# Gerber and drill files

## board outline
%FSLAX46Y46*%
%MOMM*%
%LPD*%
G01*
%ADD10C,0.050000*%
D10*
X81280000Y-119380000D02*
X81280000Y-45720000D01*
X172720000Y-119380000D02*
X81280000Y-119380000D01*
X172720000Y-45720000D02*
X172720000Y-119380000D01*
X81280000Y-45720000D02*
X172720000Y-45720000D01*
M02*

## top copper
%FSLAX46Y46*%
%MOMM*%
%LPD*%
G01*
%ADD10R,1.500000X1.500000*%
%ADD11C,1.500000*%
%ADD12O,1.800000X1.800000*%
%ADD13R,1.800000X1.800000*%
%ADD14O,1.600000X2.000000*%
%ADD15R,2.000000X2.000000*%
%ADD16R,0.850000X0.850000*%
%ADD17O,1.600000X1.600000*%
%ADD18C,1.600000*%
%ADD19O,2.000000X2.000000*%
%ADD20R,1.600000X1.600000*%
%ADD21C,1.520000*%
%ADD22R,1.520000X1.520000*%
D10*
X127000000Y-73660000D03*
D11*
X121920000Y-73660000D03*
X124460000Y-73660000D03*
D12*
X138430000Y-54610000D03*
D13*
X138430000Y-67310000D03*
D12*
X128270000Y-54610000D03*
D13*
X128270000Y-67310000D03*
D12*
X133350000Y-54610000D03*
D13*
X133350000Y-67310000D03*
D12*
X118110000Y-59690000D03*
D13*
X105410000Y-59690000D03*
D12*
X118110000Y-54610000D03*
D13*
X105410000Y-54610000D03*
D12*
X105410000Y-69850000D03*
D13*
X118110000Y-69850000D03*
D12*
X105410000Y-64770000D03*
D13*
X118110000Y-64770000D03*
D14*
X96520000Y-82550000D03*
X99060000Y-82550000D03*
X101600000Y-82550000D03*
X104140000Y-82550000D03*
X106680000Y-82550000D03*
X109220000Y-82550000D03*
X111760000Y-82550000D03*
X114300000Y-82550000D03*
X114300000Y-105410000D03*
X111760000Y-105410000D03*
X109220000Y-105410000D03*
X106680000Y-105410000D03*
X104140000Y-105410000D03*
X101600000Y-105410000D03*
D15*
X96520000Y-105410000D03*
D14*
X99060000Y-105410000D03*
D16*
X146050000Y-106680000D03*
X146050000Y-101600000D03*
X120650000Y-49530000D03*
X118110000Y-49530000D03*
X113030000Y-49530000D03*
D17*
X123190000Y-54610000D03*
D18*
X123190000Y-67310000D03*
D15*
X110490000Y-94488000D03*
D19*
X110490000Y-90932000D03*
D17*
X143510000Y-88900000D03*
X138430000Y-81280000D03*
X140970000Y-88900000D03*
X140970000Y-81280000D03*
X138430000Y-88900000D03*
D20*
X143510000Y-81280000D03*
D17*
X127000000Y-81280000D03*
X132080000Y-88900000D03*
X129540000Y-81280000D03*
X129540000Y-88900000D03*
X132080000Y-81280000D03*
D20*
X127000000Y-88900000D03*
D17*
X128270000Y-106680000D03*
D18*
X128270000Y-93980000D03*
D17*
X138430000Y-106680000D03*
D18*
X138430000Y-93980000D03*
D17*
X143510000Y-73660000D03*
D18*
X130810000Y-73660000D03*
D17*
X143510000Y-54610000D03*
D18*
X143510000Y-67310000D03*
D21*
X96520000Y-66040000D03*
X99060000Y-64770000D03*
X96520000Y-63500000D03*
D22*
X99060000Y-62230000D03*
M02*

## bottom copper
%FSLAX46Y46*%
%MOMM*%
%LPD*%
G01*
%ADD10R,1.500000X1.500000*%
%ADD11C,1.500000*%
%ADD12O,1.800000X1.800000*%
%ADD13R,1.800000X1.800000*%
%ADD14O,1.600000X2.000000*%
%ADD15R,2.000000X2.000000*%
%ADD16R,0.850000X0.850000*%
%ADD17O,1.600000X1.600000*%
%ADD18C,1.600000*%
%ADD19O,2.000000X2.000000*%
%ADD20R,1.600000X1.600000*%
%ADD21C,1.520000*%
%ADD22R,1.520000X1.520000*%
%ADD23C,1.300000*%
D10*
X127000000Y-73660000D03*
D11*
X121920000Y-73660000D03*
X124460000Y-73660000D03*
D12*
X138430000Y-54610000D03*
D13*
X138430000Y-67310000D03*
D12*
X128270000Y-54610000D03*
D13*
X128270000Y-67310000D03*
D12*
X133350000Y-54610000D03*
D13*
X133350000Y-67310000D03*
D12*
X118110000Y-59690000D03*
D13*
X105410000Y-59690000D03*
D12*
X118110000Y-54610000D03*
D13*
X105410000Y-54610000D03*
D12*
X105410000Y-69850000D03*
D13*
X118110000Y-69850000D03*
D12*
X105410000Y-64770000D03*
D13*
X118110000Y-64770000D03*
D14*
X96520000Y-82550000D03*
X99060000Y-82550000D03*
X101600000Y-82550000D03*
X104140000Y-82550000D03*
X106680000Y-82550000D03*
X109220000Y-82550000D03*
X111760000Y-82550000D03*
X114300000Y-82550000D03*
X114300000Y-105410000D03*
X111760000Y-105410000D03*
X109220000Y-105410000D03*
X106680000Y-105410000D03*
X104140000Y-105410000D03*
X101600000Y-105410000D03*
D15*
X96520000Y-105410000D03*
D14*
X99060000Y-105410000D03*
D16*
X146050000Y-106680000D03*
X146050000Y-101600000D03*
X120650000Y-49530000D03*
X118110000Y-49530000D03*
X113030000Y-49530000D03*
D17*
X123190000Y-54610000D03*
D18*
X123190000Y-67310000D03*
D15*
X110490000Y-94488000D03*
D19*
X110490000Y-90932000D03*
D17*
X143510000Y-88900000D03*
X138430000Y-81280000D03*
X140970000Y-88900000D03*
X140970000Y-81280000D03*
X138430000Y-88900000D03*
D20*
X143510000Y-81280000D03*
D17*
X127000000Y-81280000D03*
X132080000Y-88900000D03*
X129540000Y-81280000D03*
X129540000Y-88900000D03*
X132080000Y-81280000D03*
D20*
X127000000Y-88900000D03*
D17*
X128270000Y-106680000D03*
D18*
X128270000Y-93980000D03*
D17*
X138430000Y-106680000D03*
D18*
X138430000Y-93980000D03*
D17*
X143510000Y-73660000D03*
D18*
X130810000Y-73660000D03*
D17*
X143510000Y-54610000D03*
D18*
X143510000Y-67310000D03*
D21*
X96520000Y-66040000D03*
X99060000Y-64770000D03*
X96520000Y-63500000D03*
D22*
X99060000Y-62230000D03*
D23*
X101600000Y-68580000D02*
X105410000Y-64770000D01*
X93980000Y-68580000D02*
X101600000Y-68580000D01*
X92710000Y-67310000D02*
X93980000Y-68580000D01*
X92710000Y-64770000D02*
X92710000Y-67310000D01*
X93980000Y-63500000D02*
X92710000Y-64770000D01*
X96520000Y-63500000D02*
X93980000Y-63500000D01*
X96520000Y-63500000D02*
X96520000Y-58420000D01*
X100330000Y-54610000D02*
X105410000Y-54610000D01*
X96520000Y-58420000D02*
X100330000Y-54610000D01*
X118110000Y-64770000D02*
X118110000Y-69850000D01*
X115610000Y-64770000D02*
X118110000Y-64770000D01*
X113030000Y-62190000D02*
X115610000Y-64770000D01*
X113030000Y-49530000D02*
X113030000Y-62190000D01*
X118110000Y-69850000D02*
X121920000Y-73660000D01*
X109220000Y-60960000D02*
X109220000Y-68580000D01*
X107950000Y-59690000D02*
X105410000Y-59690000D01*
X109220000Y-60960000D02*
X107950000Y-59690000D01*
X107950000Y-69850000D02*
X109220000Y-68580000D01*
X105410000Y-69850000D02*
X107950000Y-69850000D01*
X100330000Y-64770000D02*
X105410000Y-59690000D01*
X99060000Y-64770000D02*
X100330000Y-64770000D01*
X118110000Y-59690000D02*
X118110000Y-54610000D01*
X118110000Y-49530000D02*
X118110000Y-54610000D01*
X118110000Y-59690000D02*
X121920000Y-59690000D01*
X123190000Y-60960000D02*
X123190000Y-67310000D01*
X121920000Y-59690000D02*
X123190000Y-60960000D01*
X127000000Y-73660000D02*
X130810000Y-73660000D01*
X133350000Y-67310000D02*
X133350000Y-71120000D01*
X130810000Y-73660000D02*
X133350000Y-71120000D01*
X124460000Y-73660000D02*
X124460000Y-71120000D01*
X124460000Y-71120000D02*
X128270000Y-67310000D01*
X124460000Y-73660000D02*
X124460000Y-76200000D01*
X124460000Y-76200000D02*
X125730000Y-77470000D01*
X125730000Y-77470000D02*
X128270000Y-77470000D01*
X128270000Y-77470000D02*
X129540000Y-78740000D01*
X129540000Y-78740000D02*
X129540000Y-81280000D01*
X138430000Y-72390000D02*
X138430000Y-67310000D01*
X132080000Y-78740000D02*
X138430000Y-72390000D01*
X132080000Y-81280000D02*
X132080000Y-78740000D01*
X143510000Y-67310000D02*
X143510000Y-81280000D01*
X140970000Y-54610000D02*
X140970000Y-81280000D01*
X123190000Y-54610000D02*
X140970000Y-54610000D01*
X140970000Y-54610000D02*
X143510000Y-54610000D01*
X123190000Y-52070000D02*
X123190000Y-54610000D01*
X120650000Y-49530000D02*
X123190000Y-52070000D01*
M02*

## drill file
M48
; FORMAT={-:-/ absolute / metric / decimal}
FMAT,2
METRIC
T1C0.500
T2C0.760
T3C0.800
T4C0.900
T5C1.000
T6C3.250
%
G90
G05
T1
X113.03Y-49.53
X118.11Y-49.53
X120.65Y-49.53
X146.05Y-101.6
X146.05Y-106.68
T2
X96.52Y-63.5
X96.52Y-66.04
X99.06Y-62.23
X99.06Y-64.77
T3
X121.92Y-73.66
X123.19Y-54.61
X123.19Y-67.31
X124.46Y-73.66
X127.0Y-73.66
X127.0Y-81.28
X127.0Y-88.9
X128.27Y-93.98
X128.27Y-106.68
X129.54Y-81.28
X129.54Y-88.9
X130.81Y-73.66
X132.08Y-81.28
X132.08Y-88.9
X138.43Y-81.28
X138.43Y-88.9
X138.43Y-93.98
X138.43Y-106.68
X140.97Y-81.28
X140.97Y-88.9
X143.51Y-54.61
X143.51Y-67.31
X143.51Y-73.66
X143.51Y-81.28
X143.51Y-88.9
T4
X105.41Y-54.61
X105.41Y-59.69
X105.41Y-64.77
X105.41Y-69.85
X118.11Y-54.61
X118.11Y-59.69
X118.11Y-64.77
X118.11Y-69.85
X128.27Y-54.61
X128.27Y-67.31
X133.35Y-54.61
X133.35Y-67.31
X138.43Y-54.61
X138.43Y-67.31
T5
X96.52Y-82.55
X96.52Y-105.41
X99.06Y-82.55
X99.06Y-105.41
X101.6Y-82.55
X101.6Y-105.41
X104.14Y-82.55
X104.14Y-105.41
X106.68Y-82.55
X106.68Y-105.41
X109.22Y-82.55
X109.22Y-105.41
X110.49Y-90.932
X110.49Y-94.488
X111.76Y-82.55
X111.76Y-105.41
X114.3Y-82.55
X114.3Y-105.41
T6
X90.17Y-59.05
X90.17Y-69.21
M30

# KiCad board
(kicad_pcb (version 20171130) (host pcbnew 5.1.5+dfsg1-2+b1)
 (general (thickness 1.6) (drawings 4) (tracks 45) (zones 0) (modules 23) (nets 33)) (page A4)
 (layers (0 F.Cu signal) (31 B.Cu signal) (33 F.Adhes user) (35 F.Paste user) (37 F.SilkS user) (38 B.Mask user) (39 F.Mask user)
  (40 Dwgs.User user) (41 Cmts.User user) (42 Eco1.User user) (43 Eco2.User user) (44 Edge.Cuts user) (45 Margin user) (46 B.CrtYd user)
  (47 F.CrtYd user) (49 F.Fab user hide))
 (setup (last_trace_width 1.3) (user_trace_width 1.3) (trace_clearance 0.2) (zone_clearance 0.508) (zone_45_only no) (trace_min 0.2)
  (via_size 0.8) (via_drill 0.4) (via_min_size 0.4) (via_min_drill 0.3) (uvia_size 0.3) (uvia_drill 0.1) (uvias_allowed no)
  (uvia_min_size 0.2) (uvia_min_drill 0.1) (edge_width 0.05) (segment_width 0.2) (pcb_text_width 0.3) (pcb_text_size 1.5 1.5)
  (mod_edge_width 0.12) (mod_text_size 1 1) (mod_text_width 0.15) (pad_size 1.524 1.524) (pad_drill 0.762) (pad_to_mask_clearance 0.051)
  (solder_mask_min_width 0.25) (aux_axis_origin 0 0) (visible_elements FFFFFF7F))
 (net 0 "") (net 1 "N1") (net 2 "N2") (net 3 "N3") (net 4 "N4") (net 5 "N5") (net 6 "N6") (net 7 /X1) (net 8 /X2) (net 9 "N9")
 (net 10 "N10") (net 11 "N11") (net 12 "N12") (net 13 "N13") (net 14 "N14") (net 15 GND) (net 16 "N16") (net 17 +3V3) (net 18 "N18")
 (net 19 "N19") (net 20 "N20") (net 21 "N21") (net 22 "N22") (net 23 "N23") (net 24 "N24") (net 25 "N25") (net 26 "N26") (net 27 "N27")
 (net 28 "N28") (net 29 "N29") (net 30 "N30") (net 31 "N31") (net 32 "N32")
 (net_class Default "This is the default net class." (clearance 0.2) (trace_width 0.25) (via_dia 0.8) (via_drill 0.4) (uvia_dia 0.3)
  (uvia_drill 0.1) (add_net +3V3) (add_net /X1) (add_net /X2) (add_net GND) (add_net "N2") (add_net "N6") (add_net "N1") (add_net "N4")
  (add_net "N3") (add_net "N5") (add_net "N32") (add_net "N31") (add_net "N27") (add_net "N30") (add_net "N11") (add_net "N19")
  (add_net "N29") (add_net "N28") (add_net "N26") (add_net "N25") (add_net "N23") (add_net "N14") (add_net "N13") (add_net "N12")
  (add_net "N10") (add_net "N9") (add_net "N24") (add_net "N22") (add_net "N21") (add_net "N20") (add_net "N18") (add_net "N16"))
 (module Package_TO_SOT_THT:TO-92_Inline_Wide (layer F.Cu) (at 127 73.66 180)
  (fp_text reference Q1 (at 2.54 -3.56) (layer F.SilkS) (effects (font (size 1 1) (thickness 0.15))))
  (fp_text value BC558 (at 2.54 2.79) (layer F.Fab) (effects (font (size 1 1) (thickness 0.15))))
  (pad 1 thru_hole rect (at 0 0 270) (size 1.5 1.5) (drill 0.8) (layers *.Cu *.Mask) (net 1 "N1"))
  (pad 3 thru_hole circle (at 5.08 0 270) (size 1.5 1.5) (drill 0.8) (layers *.Cu *.Mask) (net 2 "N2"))
  (pad 2 thru_hole circle (at 2.54 0 270) (size 1.5 1.5) (drill 0.8) (layers *.Cu *.Mask) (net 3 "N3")))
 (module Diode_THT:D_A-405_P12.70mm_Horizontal (layer F.Cu) (at 138.43 67.31 90)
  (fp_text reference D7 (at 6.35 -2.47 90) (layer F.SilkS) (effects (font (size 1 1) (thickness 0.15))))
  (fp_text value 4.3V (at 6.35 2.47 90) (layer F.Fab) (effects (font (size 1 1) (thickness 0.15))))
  (pad 2 thru_hole oval (at 12.7 0 90) (size 1.8 1.8) (drill 0.9) (layers *.Cu *.Mask) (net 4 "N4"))
  (pad 1 thru_hole rect (at 0 0 90) (size 1.8 1.8) (drill 0.9) (layers *.Cu *.Mask) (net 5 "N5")))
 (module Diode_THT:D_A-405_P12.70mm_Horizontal (layer F.Cu) (at 128.27 67.31 90)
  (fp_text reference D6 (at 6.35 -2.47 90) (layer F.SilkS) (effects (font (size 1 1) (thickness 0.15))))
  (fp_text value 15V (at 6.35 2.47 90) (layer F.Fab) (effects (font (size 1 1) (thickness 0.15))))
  (pad 2 thru_hole oval (at 12.7 0 90) (size 1.8 1.8) (drill 0.9) (layers *.Cu *.Mask) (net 4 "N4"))
  (pad 1 thru_hole rect (at 0 0 90) (size 1.8 1.8) (drill 0.9) (layers *.Cu *.Mask) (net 3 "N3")))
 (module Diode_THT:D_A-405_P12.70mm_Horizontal (layer F.Cu) (at 133.35 67.31 90)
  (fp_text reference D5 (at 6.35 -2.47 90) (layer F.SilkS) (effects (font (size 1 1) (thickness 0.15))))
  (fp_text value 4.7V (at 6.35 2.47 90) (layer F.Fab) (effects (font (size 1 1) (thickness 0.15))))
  (pad 2 thru_hole oval (at 12.7 0 90) (size 1.8 1.8) (drill 0.9) (layers *.Cu *.Mask) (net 4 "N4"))
  (pad 1 thru_hole rect (at 0 0 90) (size 1.8 1.8) (drill 0.9) (layers *.Cu *.Mask) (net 1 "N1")))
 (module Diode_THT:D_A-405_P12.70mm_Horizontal (layer F.Cu) (at 105.41 59.69)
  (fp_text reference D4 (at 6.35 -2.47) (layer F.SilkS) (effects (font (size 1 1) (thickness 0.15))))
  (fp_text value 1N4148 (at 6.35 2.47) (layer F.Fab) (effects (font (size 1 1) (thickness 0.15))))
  (pad 2 thru_hole oval (at 12.7 0) (size 1.8 1.8) (drill 0.9) (layers *.Cu *.Mask) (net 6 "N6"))
  (pad 1 thru_hole rect (at 0 0) (size 1.8 1.8) (drill 0.9) (layers *.Cu *.Mask) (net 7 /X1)))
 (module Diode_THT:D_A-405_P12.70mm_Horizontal (layer F.Cu) (at 105.41 54.61)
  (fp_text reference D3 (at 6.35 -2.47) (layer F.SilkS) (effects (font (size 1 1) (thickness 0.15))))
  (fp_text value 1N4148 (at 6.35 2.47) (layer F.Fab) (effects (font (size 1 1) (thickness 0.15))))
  (pad 2 thru_hole oval (at 12.7 0) (size 1.8 1.8) (drill 0.9) (layers *.Cu *.Mask) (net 6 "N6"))
  (pad 1 thru_hole rect (at 0 0) (size 1.8 1.8) (drill 0.9) (layers *.Cu *.Mask) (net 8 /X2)))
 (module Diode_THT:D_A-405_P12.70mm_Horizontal (layer F.Cu) (at 118.11 69.85 180)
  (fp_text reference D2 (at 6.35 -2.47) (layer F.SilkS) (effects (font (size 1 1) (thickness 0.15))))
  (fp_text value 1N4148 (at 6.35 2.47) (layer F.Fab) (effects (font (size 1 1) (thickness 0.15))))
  (pad 2 thru_hole oval (at 12.7 0 180) (size 1.8 1.8) (drill 0.9) (layers *.Cu *.Mask) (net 7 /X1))
  (pad 1 thru_hole rect (at 0 0 180) (size 1.8 1.8) (drill 0.9) (layers *.Cu *.Mask) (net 2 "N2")))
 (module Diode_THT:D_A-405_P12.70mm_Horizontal (layer F.Cu) (at 118.11 64.77 180)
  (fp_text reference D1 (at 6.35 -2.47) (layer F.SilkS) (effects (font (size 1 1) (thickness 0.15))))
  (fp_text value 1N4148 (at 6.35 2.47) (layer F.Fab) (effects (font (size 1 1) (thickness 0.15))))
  (pad 2 thru_hole oval (at 12.7 0 180) (size 1.8 1.8) (drill 0.9) (layers *.Cu *.Mask) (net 8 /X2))
  (pad 1 thru_hole rect (at 0 0 180) (size 1.8 1.8) (drill 0.9) (layers *.Cu *.Mask) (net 2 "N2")))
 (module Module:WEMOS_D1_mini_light (layer F.Cu) (at 96.52 105.41 90)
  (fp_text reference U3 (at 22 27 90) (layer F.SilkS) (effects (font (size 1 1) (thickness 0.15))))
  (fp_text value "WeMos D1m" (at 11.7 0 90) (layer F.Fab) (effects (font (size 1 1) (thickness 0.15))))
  (pad 16 thru_hole oval (at 22.86 0 90) (size 2 1.6) (drill 1) (layers *.Cu *.Mask) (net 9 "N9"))
  (pad 15 thru_hole oval (at 22.86 2.54 90) (size 2 1.6) (drill 1) (layers *.Cu *.Mask) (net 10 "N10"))
  (pad 14 thru_hole oval (at 22.86 5.08 90) (size 2 1.6) (drill 1) (layers *.Cu *.Mask) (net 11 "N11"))
  (pad 13 thru_hole oval (at 22.86 7.62 90) (size 2 1.6) (drill 1) (layers *.Cu *.Mask) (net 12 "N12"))
  (pad 12 thru_hole oval (at 22.86 10.16 90) (size 2 1.6) (drill 1) (layers *.Cu *.Mask) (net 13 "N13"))
  (pad 11 thru_hole oval (at 22.86 12.7 90) (size 2 1.6) (drill 1) (layers *.Cu *.Mask) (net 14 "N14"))
  (pad 10 thru_hole oval (at 22.86 15.24 90) (size 2 1.6) (drill 1) (layers *.Cu *.Mask) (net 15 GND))
  (pad 9 thru_hole oval (at 22.86 17.78 90) (size 2 1.6) (drill 1) (layers *.Cu *.Mask) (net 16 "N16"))
  (pad 8 thru_hole oval (at 0 17.78 90) (size 2 1.6) (drill 1) (layers *.Cu *.Mask) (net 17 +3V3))
  (pad 7 thru_hole oval (at 0 15.24 90) (size 2 1.6) (drill 1) (layers *.Cu *.Mask) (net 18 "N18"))
  (pad 6 thru_hole oval (at 0 12.7 90) (size 2 1.6) (drill 1) (layers *.Cu *.Mask) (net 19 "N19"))
  (pad 5 thru_hole oval (at 0 10.16 90) (size 2 1.6) (drill 1) (layers *.Cu *.Mask) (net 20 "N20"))
  (pad 4 thru_hole oval (at 0 7.62 90) (size 2 1.6) (drill 1) (layers *.Cu *.Mask) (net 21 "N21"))
  (pad 3 thru_hole oval (at 0 5.08 90) (size 2 1.6) (drill 1) (layers *.Cu *.Mask) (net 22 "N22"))
  (pad 1 thru_hole rect (at 0 0 90) (size 2 2) (drill 1) (layers *.Cu *.Mask) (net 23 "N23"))
  (pad 2 thru_hole oval (at 0 2.54 90) (size 2 1.6) (drill 1) (layers *.Cu *.Mask) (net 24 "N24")))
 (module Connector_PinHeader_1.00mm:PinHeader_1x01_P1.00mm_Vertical (layer F.Cu) (at 146.05 106.68)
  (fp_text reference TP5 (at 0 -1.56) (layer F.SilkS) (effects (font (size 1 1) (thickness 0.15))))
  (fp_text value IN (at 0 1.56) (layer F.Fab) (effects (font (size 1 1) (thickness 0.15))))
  (pad 1 thru_hole rect (at 0 0) (size 0.85 0.85) (drill 0.5) (layers *.Cu *.Mask) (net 19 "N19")))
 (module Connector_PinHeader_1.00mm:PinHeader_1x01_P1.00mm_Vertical (layer F.Cu) (at 146.05 101.6)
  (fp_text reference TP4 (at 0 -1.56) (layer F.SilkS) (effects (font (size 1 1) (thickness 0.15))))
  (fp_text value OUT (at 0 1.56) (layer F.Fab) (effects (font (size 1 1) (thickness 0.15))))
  (pad 1 thru_hole rect (at 0 0) (size 0.85 0.85) (drill 0.5) (layers *.Cu *.Mask) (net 11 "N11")))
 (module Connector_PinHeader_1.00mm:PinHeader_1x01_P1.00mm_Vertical (layer F.Cu) (at 120.65 49.53)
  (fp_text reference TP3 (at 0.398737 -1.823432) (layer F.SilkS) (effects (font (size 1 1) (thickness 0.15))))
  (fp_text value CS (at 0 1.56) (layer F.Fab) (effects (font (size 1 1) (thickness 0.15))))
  (pad 1 thru_hole rect (at 0 0) (size 0.85 0.85) (drill 0.5) (layers *.Cu *.Mask) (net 4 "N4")))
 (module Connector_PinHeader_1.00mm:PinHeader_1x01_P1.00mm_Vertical (layer F.Cu) (at 118.11 49.53)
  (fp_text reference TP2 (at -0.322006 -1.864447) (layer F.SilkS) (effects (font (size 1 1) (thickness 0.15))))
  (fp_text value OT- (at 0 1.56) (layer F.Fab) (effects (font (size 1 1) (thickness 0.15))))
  (pad 1 thru_hole rect (at 0 0) (size 0.85 0.85) (drill 0.5) (layers *.Cu *.Mask) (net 6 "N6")))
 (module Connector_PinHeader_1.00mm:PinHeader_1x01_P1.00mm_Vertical (layer F.Cu) (at 113.03 49.53)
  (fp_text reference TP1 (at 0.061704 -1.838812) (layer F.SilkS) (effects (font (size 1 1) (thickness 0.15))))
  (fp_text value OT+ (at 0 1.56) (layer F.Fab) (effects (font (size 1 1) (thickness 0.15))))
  (pad 1 thru_hole rect (at 0 0) (size 0.85 0.85) (drill 0.5) (layers *.Cu *.Mask) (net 2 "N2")))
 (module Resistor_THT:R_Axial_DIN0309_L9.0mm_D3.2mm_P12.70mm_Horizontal (layer F.Cu) (at 123.19 67.31 90)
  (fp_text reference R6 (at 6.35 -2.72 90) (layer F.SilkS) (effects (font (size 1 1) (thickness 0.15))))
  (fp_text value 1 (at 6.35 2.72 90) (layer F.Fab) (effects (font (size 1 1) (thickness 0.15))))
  (pad 2 thru_hole oval (at 12.7 0 90) (size 1.6 1.6) (drill 0.8) (layers *.Cu *.Mask) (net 4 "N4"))
  (pad 1 thru_hole circle (at 0 0 90) (size 1.6 1.6) (drill 0.8) (layers *.Cu *.Mask) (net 6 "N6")))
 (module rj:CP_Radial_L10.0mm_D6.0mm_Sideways (layer F.Cu) (at 110.49 92.71 180)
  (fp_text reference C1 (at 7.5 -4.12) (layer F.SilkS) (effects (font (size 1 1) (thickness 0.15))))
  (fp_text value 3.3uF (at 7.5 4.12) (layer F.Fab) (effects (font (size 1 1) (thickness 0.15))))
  (pad 1 thru_hole rect (at 0 -1.778 180) (size 2 2) (drill 1) (layers *.Cu *.Mask) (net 17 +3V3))
  (pad 2 thru_hole oval (at 0 1.778 180) (size 2 2) (drill 1) (layers *.Cu *.Mask) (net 15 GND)))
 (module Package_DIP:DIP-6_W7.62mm (layer F.Cu) (at 143.51 81.28 270)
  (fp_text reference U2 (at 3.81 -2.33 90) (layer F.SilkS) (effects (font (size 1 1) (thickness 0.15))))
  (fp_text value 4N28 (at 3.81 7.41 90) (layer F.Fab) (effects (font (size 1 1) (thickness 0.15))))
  (pad 6 thru_hole oval (at 7.62 0 270) (size 1.6 1.6) (drill 0.8) (layers *.Cu *.Mask) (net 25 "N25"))
  (pad 3 thru_hole oval (at 0 5.08 270) (size 1.6 1.6) (drill 0.8) (layers *.Cu *.Mask) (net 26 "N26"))
  (pad 5 thru_hole oval (at 7.62 2.54 270) (size 1.6 1.6) (drill 0.8) (layers *.Cu *.Mask) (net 17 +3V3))
  (pad 2 thru_hole oval (at 0 2.54 270) (size 1.6 1.6) (drill 0.8) (layers *.Cu *.Mask) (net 4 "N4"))
  (pad 4 thru_hole oval (at 7.62 5.08 270) (size 1.6 1.6) (drill 0.8) (layers *.Cu *.Mask) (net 19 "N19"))
  (pad 1 thru_hole rect (at 0 0 270) (size 1.6 1.6) (drill 0.8) (layers *.Cu *.Mask) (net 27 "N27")))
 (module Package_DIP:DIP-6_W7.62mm (layer F.Cu) (at 127 88.9 90)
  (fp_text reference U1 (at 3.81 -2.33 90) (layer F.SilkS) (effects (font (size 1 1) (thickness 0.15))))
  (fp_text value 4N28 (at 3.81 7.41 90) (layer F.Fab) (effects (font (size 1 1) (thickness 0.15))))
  (pad 6 thru_hole oval (at 7.62 0 90) (size 1.6 1.6) (drill 0.8) (layers *.Cu *.Mask) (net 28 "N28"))
  (pad 3 thru_hole oval (at 0 5.08 90) (size 1.6 1.6) (drill 0.8) (layers *.Cu *.Mask) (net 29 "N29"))
  (pad 5 thru_hole oval (at 7.62 2.54 90) (size 1.6 1.6) (drill 0.8) (layers *.Cu *.Mask) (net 3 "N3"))
  (pad 2 thru_hole oval (at 0 2.54 90) (size 1.6 1.6) (drill 0.8) (layers *.Cu *.Mask) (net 15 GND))
  (pad 4 thru_hole oval (at 7.62 5.08 90) (size 1.6 1.6) (drill 0.8) (layers *.Cu *.Mask) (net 5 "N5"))
  (pad 1 thru_hole rect (at 0 0 90) (size 1.6 1.6) (drill 0.8) (layers *.Cu *.Mask) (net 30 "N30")))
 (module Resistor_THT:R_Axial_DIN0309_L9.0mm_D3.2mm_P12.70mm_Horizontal (layer F.Cu) (at 128.27 93.98 270)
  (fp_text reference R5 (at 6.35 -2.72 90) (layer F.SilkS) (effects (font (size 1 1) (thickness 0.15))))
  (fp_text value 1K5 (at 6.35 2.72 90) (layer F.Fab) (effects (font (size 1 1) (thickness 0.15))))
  (pad 2 thru_hole oval (at 12.7 0 270) (size 1.6 1.6) (drill 0.8) (layers *.Cu *.Mask) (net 19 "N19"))
  (pad 1 thru_hole circle (at 0 0 270) (size 1.6 1.6) (drill 0.8) (layers *.Cu *.Mask) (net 15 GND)))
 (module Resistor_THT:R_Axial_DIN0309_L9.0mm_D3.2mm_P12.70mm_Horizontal (layer F.Cu) (at 138.43 93.98 270)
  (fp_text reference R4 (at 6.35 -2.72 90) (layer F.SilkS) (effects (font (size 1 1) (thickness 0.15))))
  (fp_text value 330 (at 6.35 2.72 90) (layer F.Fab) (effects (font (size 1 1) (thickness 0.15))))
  (pad 2 thru_hole oval (at 12.7 0 270) (size 1.6 1.6) (drill 0.8) (layers *.Cu *.Mask) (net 11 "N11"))
  (pad 1 thru_hole circle (at 0 0 270) (size 1.6 1.6) (drill 0.8) (layers *.Cu *.Mask) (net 30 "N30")))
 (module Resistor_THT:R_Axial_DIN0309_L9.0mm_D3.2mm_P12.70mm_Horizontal (layer F.Cu) (at 130.81 73.66)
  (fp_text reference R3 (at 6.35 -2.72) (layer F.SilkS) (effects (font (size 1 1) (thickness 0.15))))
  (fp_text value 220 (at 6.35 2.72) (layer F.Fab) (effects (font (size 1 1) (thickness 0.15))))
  (pad 2 thru_hole oval (at 12.7 0) (size 1.6 1.6) (drill 0.8) (layers *.Cu *.Mask) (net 27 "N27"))
  (pad 1 thru_hole circle (at 0 0) (size 1.6 1.6) (drill 0.8) (layers *.Cu *.Mask) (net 1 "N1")))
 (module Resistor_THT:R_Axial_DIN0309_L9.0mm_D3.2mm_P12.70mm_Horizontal (layer F.Cu) (at 143.51 67.31 90)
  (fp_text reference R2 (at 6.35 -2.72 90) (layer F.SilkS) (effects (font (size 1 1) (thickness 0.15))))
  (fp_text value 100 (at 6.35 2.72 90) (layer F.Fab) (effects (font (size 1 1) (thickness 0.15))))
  (pad 2 thru_hole oval (at 12.7 0 90) (size 1.6 1.6) (drill 0.8) (layers *.Cu *.Mask) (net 4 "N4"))
  (pad 1 thru_hole circle (at 0 0 90) (size 1.6 1.6) (drill 0.8) (layers *.Cu *.Mask) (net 27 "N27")))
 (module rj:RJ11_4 (layer F.Cu) (at 99.06 60.96 270)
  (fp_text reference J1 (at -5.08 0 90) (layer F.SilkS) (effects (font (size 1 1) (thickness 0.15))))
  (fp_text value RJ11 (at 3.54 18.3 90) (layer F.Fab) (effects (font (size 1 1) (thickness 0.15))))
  (pad "" np_thru_hole circle (at 8.25 8.89 270) (size 3.25 3.25) (drill 3.25) (layers *.Cu *.Mask))
  (pad 4 thru_hole circle (at 5.08 2.54 270) (size 1.52 1.52) (drill 0.76) (layers *.Cu *.Mask) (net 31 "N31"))
  (pad 3 thru_hole circle (at 3.81 0 270) (size 1.52 1.52) (drill 0.76) (layers *.Cu *.Mask) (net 7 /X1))
  (pad 2 thru_hole circle (at 2.54 2.54 270) (size 1.52 1.52) (drill 0.76) (layers *.Cu *.Mask) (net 8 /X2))
  (pad "" np_thru_hole circle (at -1.91 8.89 270) (size 3.25 3.25) (drill 3.25) (layers *.Cu *.Mask))
  (pad 1 thru_hole rect (at 1.27 0 270) (size 1.52 1.52) (drill 0.76) (layers *.Cu *.Mask) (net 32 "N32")))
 (gr_line (start 81.28 119.38) (end 81.28 45.72) (layer Edge.Cuts) (width 0.05))
 (gr_line (start 172.72 119.38) (end 81.28 119.38) (layer Edge.Cuts) (width 0.05))
 (gr_line (start 172.72 45.72) (end 172.72 119.38) (layer Edge.Cuts) (width 0.05))
 (gr_line (start 81.28 45.72) (end 172.72 45.72) (layer Edge.Cuts) (width 0.05))
 (segment (start 101.6 68.58) (end 105.41 64.77) (width 1.3) (layer B.Cu) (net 8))
 (segment (start 93.98 68.58) (end 101.6 68.58) (width 1.3) (layer B.Cu) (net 8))
 (segment (start 92.71 67.31) (end 93.98 68.58) (width 1.3) (layer B.Cu) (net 8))
 (segment (start 92.71 64.77) (end 92.71 67.31) (width 1.3) (layer B.Cu) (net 8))
 (segment (start 93.98 63.5) (end 92.71 64.77) (width 1.3) (layer B.Cu) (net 8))
 (segment (start 96.52 63.5) (end 93.98 63.5) (width 1.3) (layer B.Cu) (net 8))
 (segment (start 96.52 63.5) (end 96.52 58.42) (width 1.3) (layer B.Cu) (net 8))
 (segment (start 100.33 54.61) (end 105.41 54.61) (width 1.3) (layer B.Cu) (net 8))
 (segment (start 96.52 58.42) (end 100.33 54.61) (width 1.3) (layer B.Cu) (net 8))
 (segment (start 118.11 64.77) (end 118.11 69.85) (width 1.3) (layer B.Cu) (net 2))
 (segment (start 115.61 64.77) (end 118.11 64.77) (width 1.3) (layer B.Cu) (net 2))
 (segment (start 113.03 62.19) (end 115.61 64.77) (width 1.3) (layer B.Cu) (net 2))
 (segment (start 113.03 49.53) (end 113.03 62.19) (width 1.3) (layer B.Cu) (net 2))
 (segment (start 118.11 69.85) (end 121.92 73.66) (width 1.3) (layer B.Cu) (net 2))
 (segment (start 109.22 60.96) (end 109.22 68.58) (width 1.3) (layer B.Cu) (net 7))
 (segment (start 107.95 59.69) (end 105.41 59.69) (width 1.3) (layer B.Cu) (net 7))
 (segment (start 109.22 60.96) (end 107.95 59.69) (width 1.3) (layer B.Cu) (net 7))
 (segment (start 107.95 69.85) (end 109.22 68.58) (width 1.3) (layer B.Cu) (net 7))
 (segment (start 105.41 69.85) (end 107.95 69.85) (width 1.3) (layer B.Cu) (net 7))
 (segment (start 100.33 64.77) (end 105.41 59.69) (width 1.3) (layer B.Cu) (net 7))
 (segment (start 99.06 64.77) (end 100.33 64.77) (width 1.3) (layer B.Cu) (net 7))
 (segment (start 118.11 59.69) (end 118.11 54.61) (width 1.3) (layer B.Cu) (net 6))
 (segment (start 118.11 49.53) (end 118.11 54.61) (width 1.3) (layer B.Cu) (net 6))
 (segment (start 118.11 59.69) (end 121.92 59.69) (width 1.3) (layer B.Cu) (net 6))
 (segment (start 123.19 60.96) (end 123.19 67.31) (width 1.3) (layer B.Cu) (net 6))
 (segment (start 121.92 59.69) (end 123.19 60.96) (width 1.3) (layer B.Cu) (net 6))
 (segment (start 127 73.66) (end 130.81 73.66) (width 1.3) (layer B.Cu) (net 1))
 (segment (start 133.35 67.31) (end 133.35 71.12) (width 1.3) (layer B.Cu) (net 1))
 (segment (start 130.81 73.66) (end 133.35 71.12) (width 1.3) (layer B.Cu) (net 1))
 (segment (start 124.46 73.66) (end 124.46 71.12) (width 1.3) (layer B.Cu) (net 3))
 (segment (start 124.46 71.12) (end 128.27 67.31) (width 1.3) (layer B.Cu) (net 3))
 (segment (start 124.46 73.66) (end 124.46 76.2) (width 1.3) (layer B.Cu) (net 3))
 (segment (start 124.46 76.2) (end 125.73 77.47) (width 1.3) (layer B.Cu) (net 3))
 (segment (start 125.73 77.47) (end 128.27 77.47) (width 1.3) (layer B.Cu) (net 3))
 (segment (start 128.27 77.47) (end 129.54 78.74) (width 1.3) (layer B.Cu) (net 3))
 (segment (start 129.54 78.74) (end 129.54 81.28) (width 1.3) (layer B.Cu) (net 3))
 (segment (start 138.43 72.39) (end 138.43 67.31) (width 1.3) (layer B.Cu) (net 5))
 (segment (start 132.08 78.74) (end 138.43 72.39) (width 1.3) (layer B.Cu) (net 5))
 (segment (start 132.08 81.28) (end 132.08 78.74) (width 1.3) (layer B.Cu) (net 5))
 (segment (start 143.51 67.31) (end 143.51 81.28) (width 1.3) (layer B.Cu) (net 27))
 (segment (start 140.97 54.61) (end 140.97 81.28) (width 1.3) (layer B.Cu) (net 4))
 (segment (start 123.19 54.61) (end 140.97 54.61) (width 1.3) (layer B.Cu) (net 4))
 (segment (start 140.97 54.61) (end 143.51 54.61) (width 1.3) (layer B.Cu) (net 4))
 (segment (start 123.19 52.07) (end 123.19 54.61) (width 1.3) (layer B.Cu) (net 4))
 (segment (start 120.65 49.53) (end 123.19 52.07) (width 1.3) (layer B.Cu) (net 4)))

